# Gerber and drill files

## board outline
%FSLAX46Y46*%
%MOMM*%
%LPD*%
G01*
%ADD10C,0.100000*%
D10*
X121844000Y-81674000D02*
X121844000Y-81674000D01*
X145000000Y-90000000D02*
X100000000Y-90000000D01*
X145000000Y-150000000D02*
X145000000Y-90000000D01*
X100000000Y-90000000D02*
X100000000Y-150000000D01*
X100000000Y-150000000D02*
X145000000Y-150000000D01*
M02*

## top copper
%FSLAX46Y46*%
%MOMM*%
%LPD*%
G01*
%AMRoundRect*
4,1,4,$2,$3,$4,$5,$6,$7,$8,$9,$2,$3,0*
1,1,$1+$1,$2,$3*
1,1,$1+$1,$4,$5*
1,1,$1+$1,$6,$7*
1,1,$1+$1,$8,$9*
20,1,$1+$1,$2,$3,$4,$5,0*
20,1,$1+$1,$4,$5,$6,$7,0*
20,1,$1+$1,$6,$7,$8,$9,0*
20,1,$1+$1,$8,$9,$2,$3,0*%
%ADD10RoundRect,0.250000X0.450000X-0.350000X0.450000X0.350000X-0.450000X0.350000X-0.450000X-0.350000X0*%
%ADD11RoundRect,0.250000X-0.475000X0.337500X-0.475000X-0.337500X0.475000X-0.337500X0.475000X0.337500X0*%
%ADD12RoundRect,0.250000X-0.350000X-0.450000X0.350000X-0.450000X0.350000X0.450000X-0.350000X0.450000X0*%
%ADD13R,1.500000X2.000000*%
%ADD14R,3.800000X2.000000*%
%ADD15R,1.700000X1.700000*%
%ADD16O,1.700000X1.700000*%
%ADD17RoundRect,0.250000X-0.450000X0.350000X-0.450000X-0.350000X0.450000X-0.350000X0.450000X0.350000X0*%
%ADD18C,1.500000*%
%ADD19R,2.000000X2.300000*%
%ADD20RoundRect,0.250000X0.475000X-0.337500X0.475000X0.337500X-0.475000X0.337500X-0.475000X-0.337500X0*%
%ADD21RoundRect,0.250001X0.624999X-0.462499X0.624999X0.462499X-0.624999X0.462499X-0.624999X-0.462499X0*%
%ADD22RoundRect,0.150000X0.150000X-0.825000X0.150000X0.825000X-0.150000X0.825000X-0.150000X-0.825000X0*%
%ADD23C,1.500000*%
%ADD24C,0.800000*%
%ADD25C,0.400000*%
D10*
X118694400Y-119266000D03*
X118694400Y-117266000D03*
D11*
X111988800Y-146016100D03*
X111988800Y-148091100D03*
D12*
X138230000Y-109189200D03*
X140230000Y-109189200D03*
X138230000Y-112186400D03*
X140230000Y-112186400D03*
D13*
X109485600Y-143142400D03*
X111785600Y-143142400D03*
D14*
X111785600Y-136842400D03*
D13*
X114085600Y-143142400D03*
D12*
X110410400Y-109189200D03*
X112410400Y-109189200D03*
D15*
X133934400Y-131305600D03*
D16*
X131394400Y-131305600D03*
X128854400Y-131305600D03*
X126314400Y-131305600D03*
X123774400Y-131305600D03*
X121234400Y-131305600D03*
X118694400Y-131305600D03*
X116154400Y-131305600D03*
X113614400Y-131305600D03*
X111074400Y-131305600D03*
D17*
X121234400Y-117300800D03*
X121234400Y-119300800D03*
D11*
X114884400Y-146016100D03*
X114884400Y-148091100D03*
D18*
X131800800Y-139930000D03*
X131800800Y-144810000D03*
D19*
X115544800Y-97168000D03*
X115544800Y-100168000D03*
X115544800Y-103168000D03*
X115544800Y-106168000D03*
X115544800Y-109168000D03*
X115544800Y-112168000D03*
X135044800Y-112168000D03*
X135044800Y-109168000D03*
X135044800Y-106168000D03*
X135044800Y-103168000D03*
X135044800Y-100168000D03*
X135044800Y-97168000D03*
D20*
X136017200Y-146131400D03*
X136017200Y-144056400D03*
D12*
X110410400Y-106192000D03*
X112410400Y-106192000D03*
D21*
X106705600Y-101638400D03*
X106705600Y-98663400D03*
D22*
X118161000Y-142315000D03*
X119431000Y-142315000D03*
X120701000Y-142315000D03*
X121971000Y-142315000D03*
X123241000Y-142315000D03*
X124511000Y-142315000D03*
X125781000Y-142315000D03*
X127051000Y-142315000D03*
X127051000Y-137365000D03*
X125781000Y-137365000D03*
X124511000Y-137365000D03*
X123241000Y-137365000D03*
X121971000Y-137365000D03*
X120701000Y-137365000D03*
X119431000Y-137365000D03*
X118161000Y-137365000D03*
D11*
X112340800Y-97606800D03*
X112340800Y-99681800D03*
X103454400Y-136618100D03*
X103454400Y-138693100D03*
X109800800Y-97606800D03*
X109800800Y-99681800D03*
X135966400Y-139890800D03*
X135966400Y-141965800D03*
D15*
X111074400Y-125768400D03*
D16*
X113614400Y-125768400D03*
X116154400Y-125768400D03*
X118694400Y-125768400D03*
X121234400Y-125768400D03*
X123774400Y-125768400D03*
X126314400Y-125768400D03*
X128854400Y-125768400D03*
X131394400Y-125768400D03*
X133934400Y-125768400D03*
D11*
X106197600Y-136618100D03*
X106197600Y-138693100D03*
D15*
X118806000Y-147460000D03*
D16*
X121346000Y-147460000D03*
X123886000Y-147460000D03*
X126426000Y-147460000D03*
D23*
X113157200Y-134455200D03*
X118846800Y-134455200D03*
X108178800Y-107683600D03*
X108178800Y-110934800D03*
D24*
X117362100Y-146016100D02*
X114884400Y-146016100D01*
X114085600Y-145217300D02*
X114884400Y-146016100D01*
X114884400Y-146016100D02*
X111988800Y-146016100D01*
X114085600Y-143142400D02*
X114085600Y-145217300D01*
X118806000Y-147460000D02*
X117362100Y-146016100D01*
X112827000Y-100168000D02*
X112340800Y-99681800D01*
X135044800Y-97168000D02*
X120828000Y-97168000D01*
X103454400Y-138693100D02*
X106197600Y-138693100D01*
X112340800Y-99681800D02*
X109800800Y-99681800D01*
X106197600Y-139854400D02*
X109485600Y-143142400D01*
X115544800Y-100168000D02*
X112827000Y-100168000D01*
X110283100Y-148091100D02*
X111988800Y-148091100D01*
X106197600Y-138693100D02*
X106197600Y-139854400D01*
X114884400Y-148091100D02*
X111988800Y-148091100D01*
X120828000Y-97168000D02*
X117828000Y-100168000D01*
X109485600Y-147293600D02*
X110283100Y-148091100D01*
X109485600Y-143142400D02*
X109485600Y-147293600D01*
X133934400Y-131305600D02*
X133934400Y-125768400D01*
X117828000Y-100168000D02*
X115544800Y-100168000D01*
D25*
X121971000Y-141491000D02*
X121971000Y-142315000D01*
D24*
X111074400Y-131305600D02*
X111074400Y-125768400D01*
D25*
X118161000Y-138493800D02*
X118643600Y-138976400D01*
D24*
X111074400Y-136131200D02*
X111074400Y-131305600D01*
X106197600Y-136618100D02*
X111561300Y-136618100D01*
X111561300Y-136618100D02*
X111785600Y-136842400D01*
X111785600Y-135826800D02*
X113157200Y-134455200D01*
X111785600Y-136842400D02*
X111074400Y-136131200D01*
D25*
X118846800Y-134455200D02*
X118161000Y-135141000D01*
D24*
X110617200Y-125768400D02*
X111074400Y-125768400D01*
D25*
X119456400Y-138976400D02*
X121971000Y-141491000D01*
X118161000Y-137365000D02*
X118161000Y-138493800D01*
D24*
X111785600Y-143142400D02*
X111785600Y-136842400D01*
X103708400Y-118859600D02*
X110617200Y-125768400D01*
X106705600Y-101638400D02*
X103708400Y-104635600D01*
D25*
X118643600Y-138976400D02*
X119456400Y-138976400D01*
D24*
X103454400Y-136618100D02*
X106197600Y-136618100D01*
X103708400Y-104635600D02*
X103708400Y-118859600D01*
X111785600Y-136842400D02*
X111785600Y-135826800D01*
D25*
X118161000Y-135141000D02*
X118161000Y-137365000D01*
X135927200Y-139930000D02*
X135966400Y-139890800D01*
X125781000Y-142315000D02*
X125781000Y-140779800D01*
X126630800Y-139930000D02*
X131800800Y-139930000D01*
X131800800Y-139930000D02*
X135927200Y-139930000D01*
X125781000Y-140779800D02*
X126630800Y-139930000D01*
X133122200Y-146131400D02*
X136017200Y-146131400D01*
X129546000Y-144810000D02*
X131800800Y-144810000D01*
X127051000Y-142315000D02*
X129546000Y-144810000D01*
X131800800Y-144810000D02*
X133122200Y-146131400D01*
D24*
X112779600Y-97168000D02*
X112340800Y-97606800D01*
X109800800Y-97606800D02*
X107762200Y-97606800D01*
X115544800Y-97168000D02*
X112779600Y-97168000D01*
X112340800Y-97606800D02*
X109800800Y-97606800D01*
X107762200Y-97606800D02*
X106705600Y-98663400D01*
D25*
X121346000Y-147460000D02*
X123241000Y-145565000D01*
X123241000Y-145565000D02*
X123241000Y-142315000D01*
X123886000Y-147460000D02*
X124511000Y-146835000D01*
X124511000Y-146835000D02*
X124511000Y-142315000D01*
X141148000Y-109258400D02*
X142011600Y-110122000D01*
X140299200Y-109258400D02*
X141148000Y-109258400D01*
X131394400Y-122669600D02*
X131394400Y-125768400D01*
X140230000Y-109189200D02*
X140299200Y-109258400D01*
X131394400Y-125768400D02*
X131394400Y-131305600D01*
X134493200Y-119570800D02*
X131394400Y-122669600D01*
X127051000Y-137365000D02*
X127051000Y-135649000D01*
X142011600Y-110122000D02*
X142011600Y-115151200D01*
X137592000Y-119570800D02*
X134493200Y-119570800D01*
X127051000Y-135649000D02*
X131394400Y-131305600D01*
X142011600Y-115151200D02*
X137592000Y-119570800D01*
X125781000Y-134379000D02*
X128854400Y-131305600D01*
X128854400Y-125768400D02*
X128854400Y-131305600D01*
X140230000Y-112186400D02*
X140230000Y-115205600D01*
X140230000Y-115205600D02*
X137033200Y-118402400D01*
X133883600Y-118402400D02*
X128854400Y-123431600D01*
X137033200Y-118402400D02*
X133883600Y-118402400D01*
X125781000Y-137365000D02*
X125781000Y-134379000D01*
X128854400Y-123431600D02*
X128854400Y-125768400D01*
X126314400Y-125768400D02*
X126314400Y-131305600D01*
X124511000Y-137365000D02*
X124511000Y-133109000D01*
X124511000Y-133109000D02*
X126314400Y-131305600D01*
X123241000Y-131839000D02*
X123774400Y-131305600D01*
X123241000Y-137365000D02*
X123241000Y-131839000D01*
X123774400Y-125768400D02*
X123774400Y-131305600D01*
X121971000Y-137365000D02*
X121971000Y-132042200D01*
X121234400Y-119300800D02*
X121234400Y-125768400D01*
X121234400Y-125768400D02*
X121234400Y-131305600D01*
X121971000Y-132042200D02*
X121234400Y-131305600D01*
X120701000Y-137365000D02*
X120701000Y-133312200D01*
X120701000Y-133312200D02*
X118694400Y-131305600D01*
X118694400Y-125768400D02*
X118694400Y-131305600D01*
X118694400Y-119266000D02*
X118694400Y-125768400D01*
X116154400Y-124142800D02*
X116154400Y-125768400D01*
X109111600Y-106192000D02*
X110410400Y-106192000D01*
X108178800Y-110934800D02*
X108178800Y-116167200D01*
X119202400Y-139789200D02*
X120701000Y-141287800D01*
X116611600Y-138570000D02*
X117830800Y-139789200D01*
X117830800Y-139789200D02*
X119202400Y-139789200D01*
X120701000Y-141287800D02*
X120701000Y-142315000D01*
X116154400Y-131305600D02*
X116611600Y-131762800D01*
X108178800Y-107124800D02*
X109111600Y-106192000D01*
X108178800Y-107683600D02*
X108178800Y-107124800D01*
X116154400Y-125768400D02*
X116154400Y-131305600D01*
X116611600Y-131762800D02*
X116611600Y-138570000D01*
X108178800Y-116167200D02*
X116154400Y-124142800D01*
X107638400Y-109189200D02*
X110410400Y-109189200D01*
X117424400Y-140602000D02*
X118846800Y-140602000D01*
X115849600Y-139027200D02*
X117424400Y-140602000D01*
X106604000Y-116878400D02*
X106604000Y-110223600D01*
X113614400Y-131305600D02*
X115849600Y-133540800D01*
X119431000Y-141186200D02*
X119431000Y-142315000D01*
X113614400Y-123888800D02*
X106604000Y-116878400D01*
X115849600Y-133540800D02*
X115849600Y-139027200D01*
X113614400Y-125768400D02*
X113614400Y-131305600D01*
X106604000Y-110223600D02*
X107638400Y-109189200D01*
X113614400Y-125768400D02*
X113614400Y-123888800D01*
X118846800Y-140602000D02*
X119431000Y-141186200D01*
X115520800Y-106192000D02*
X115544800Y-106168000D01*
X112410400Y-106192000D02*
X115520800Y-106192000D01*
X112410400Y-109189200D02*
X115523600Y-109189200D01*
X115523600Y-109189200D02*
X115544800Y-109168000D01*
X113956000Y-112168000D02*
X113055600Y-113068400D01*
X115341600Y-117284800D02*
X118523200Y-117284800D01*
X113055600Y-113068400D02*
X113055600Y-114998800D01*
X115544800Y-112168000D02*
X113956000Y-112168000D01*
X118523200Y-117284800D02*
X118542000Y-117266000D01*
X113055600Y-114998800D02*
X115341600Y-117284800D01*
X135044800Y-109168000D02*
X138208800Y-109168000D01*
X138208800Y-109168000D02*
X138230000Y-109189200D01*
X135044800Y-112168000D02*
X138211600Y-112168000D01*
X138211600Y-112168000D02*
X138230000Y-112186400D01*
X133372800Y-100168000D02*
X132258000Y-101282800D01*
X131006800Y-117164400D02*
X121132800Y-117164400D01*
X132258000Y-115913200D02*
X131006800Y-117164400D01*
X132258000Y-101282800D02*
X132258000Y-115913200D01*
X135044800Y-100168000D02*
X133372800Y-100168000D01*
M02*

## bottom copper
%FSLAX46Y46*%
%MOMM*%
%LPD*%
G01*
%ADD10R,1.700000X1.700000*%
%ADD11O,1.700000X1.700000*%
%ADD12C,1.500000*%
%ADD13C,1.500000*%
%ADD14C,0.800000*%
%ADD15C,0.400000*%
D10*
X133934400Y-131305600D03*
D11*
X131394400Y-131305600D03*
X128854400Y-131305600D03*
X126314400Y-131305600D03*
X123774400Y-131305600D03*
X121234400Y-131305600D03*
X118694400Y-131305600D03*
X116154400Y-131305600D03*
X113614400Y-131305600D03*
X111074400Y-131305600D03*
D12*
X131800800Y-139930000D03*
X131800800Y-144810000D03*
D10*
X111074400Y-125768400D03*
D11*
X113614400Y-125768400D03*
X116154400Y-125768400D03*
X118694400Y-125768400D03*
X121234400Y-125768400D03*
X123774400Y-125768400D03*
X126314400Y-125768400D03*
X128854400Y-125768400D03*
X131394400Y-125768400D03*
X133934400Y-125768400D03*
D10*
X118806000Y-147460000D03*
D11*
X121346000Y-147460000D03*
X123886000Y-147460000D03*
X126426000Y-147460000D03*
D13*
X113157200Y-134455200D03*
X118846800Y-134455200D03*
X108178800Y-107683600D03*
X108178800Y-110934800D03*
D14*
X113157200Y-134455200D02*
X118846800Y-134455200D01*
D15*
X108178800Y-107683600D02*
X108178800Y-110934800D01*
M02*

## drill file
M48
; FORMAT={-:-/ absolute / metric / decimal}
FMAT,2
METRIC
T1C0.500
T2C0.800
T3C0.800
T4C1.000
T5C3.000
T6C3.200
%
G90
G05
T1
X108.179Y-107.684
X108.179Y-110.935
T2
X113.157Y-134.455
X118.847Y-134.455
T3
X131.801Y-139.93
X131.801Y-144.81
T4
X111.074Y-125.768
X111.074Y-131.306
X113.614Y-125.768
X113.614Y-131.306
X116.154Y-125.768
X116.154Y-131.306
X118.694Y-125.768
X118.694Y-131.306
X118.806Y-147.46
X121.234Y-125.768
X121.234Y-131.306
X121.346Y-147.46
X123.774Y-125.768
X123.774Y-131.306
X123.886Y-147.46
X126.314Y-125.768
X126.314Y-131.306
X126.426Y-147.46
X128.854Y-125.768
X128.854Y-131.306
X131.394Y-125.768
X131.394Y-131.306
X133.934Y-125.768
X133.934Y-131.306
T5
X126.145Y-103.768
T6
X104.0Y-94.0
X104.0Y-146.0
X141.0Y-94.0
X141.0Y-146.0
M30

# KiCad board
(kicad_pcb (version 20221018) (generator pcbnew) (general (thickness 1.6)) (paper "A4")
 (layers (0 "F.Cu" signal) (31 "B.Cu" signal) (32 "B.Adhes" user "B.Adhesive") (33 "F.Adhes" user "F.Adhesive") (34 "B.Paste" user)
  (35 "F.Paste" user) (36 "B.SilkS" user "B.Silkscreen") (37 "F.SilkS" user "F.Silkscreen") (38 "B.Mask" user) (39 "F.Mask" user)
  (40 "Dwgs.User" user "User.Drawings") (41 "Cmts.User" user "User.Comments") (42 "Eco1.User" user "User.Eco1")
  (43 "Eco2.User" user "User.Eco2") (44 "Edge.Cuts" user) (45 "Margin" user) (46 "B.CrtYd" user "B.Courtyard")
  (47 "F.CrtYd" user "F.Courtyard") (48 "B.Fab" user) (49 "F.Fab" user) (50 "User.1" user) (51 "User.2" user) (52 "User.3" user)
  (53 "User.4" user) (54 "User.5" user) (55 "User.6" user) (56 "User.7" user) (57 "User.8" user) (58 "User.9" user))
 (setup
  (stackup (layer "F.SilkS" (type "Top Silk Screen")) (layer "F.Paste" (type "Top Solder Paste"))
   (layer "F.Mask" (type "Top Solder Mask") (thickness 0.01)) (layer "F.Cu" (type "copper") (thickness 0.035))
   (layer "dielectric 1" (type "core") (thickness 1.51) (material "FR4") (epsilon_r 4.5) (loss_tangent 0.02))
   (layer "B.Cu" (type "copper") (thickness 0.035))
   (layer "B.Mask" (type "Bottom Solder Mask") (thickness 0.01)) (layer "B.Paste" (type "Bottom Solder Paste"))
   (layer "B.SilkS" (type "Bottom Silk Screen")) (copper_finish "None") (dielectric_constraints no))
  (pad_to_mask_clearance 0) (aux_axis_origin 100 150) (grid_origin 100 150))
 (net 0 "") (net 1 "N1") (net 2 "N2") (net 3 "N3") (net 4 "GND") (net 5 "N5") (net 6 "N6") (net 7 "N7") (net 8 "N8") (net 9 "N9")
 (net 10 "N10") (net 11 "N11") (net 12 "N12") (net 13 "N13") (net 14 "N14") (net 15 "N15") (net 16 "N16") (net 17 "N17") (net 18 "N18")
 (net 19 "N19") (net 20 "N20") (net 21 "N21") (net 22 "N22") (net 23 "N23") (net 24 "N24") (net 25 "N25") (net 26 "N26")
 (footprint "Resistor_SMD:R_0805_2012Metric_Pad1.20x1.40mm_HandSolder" (layer "F.Cu") (at 118.6944 118.266 90)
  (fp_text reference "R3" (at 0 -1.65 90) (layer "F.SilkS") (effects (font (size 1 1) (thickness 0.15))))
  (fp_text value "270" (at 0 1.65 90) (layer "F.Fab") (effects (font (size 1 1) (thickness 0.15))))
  (pad "1" smd roundrect (at -1 0 90) (size 1.2 1.4) (layers "F.Cu" "F.Paste" "F.Mask") (roundrect_rratio 0.208333) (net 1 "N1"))
  (pad "2" smd roundrect (at 1 0 90) (size 1.2 1.4) (layers "F.Cu" "F.Paste" "F.Mask") (roundrect_rratio 0.208333) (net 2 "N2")))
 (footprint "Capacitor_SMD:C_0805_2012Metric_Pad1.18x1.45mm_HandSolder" (layer "F.Cu") (at 111.9888 147.0536 -90)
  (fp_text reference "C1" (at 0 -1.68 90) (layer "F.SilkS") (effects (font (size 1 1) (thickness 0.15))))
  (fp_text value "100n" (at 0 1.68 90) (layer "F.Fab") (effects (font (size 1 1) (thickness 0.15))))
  (pad "1" smd roundrect (at -1.0375 0 270) (size 1.175 1.45) (layers "F.Cu" "F.Paste" "F.Mask") (roundrect_rratio 0.212766) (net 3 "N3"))
  (pad "2" smd roundrect (at 1.0375 0 270) (size 1.175 1.45) (layers "F.Cu" "F.Paste" "F.Mask") (roundrect_rratio 0.212766) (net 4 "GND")))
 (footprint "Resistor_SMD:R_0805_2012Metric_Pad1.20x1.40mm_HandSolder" (layer "F.Cu") (at 139.23 109.1892)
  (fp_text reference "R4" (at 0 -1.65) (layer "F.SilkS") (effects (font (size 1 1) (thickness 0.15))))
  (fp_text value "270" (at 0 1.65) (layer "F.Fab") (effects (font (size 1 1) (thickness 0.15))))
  (pad "1" smd roundrect (at -1 0) (size 1.2 1.4) (layers "F.Cu" "F.Paste" "F.Mask") (roundrect_rratio 0.208333) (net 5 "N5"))
  (pad "2" smd roundrect (at 1 0) (size 1.2 1.4) (layers "F.Cu" "F.Paste" "F.Mask") (roundrect_rratio 0.208333) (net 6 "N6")))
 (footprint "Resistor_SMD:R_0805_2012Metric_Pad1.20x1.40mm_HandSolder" (layer "F.Cu") (at 139.23 112.1864)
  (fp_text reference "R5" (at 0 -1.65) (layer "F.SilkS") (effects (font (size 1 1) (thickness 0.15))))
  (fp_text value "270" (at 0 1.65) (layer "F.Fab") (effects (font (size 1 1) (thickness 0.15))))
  (pad "1" smd roundrect (at -1 0) (size 1.2 1.4) (layers "F.Cu" "F.Paste" "F.Mask") (roundrect_rratio 0.208333) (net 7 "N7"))
  (pad "2" smd roundrect (at 1 0) (size 1.2 1.4) (layers "F.Cu" "F.Paste" "F.Mask") (roundrect_rratio 0.208333) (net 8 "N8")))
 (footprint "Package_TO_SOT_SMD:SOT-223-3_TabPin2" (layer "F.Cu") (at 111.7856 139.9924 90)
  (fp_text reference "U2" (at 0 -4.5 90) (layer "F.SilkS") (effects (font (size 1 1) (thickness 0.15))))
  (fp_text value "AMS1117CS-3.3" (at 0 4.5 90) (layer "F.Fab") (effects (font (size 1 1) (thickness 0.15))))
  (pad "1" smd rect (at -3.15 -2.3 90) (size 2 1.5) (layers "F.Cu" "F.Paste" "F.Mask") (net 4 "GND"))
  (pad "2" smd rect (at -3.15 0 90) (size 2 1.5) (layers "F.Cu" "F.Paste" "F.Mask") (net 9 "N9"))
  (pad "2" smd rect (at 3.15 0 90) (size 2 3.8) (layers "F.Cu" "F.Paste" "F.Mask") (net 9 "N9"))
  (pad "3" smd rect (at -3.15 2.3 90) (size 2 1.5) (layers "F.Cu" "F.Paste" "F.Mask") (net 3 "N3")))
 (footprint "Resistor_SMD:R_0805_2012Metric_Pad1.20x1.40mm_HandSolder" (layer "F.Cu") (at 111.4104 109.1892)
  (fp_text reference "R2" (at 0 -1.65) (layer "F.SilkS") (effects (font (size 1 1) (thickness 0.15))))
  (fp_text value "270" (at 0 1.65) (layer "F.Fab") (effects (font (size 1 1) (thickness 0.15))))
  (pad "1" smd roundrect (at -1 0) (size 1.2 1.4) (layers "F.Cu" "F.Paste" "F.Mask") (roundrect_rratio 0.208333) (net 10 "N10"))
  (pad "2" smd roundrect (at 1 0) (size 1.2 1.4) (layers "F.Cu" "F.Paste" "F.Mask") (roundrect_rratio 0.208333) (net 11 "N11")))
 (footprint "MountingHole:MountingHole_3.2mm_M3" (layer "F.Cu") (at 141 146)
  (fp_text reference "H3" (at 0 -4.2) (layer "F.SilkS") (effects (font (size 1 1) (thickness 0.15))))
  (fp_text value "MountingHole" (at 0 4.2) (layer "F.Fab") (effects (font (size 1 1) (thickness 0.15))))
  (pad "" np_thru_hole circle (at 0 0) (size 3.2 3.2) (drill 3.2) (layers "*.Cu" "*.Mask")))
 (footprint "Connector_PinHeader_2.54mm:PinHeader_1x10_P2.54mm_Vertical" (layer "F.Cu") (at 133.9344 131.3056 -90)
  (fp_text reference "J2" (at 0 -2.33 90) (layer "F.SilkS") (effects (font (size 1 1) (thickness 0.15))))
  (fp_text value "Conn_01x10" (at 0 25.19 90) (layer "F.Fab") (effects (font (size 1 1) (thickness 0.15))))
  (pad "1" thru_hole rect (at 0 0 270) (size 1.7 1.7) (drill 1) (layers "*.Cu" "*.Mask") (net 4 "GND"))
  (pad "2" thru_hole oval (at 0 2.54 270) (size 1.7 1.7) (drill 1) (layers "*.Cu" "*.Mask") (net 6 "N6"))
  (pad "3" thru_hole oval (at 0 5.08 270) (size 1.7 1.7) (drill 1) (layers "*.Cu" "*.Mask") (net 8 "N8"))
  (pad "4" thru_hole oval (at 0 7.62 270) (size 1.7 1.7) (drill 1) (layers "*.Cu" "*.Mask") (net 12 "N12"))
  (pad "5" thru_hole oval (at 0 10.16 270) (size 1.7 1.7) (drill 1) (layers "*.Cu" "*.Mask") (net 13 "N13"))
  (pad "6" thru_hole oval (at 0 12.7 270) (size 1.7 1.7) (drill 1) (layers "*.Cu" "*.Mask") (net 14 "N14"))
  (pad "7" thru_hole oval (at 0 15.24 270) (size 1.7 1.7) (drill 1) (layers "*.Cu" "*.Mask") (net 1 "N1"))
  (pad "8" thru_hole oval (at 0 17.78 270) (size 1.7 1.7) (drill 1) (layers "*.Cu" "*.Mask") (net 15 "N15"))
  (pad "9" thru_hole oval (at 0 20.32 270) (size 1.7 1.7) (drill 1) (layers "*.Cu" "*.Mask") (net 10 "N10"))
  (pad "10" thru_hole oval (at 0 22.86 270) (size 1.7 1.7) (drill 1) (layers "*.Cu" "*.Mask") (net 9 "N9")))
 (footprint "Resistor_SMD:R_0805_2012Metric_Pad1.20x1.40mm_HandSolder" (layer "F.Cu") (at 121.2344 118.3008 -90)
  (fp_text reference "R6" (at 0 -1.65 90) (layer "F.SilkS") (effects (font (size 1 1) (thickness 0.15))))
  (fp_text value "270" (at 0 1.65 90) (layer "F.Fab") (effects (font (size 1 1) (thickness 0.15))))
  (pad "1" smd roundrect (at -1 0 270) (size 1.2 1.4) (layers "F.Cu" "F.Paste" "F.Mask") (roundrect_rratio 0.208333) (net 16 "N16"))
  (pad "2" smd roundrect (at 1 0 270) (size 1.2 1.4) (layers "F.Cu" "F.Paste" "F.Mask") (roundrect_rratio 0.208333) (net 14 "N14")))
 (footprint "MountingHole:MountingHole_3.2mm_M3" (layer "F.Cu") (at 104 94)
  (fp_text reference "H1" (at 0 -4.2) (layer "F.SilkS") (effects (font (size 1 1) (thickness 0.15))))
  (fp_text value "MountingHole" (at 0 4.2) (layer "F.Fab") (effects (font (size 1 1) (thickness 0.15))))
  (pad "" np_thru_hole circle (at 0 0) (size 3.2 3.2) (drill 3.2) (layers "*.Cu" "*.Mask")))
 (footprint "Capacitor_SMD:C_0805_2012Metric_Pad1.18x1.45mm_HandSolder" (layer "F.Cu") (at 114.8844 147.0536 -90)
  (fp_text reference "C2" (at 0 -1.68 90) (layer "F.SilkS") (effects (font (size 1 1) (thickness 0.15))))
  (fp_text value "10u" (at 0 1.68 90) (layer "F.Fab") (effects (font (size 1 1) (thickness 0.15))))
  (pad "1" smd roundrect (at -1.0375 0 270) (size 1.175 1.45) (layers "F.Cu" "F.Paste" "F.Mask") (roundrect_rratio 0.212766) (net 3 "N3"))
  (pad "2" smd roundrect (at 1.0375 0 270) (size 1.175 1.45) (layers "F.Cu" "F.Paste" "F.Mask") (roundrect_rratio 0.212766) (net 4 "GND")))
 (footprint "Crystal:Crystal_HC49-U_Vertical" (layer "F.Cu") (at 131.8008 139.93 -90)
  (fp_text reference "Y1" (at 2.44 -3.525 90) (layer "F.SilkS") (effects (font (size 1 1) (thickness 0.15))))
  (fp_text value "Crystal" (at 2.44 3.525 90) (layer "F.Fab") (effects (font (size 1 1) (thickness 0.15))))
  (pad "1" thru_hole circle (at 0 0 270) (size 1.5 1.5) (drill 0.8) (layers "*.Cu" "*.Mask") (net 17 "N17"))
  (pad "2" thru_hole circle (at 4.88 0 270) (size 1.5 1.5) (drill 0.8) (layers "*.Cu" "*.Mask") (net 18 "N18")))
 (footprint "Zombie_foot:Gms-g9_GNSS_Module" (layer "F.Cu") (at 125.2948 104.668)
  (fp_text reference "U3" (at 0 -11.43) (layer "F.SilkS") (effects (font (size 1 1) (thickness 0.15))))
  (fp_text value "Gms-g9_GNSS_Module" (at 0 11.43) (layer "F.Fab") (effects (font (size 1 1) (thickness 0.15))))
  (pad "" np_thru_hole circle (at 0.85 -0.9) (size 3 3) (drill 3) (layers "*.Cu" "*.Mask"))
  (pad "1" smd rect (at -9.75 -7.5) (size 2 2.3) (layers "F.Cu" "F.Paste" "F.Mask") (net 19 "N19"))
  (pad "2" smd rect (at -9.75 -4.5) (size 2 2.3) (layers "F.Cu" "F.Paste" "F.Mask") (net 4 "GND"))
  (pad "3" smd rect (at -9.75 -1.5) (size 2 2.3) (layers "F.Cu" "F.Paste" "F.Mask") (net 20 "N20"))
  (pad "4" smd rect (at -9.75 1.5) (size 2 2.3) (layers "F.Cu" "F.Paste" "F.Mask") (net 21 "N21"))
  (pad "5" smd rect (at -9.75 4.5) (size 2 2.3) (layers "F.Cu" "F.Paste" "F.Mask") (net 11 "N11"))
  (pad "6" smd rect (at -9.75 7.5) (size 2 2.3) (layers "F.Cu" "F.Paste" "F.Mask") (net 2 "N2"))
  (pad "7" smd rect (at 9.75 7.5) (size 2 2.3) (layers "F.Cu" "F.Paste" "F.Mask") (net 7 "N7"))
  (pad "8" smd rect (at 9.75 4.5) (size 2 2.3) (layers "F.Cu" "F.Paste" "F.Mask") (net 5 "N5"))
  (pad "9" smd rect (at 9.75 1.5) (size 2 2.3) (layers "F.Cu" "F.Paste" "F.Mask") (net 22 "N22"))
  (pad "10" smd rect (at 9.75 -1.5) (size 2 2.3) (layers "F.Cu" "F.Paste" "F.Mask") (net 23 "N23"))
  (pad "11" smd rect (at 9.75 -4.5) (size 2 2.3) (layers "F.Cu" "F.Paste" "F.Mask") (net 16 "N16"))
  (pad "12" smd rect (at 9.75 -7.5) (size 2 2.3) (layers "F.Cu" "F.Paste" "F.Mask") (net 4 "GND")))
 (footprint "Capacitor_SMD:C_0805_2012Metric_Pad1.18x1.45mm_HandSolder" (layer "F.Cu") (at 136.0172 145.0939 90)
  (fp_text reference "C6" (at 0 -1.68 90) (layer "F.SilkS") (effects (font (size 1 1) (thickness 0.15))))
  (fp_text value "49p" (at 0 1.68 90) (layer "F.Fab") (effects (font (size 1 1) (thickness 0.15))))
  (pad "1" smd roundrect (at -1.0375 0 90) (size 1.175 1.45) (layers "F.Cu" "F.Paste" "F.Mask") (roundrect_rratio 0.212766) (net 18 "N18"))
  (pad "2" smd roundrect (at 1.0375 0 90) (size 1.175 1.45) (layers "F.Cu" "F.Paste" "F.Mask") (roundrect_rratio 0.212766) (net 4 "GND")))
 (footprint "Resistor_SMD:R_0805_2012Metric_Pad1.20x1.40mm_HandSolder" (layer "F.Cu") (at 111.4104 106.192)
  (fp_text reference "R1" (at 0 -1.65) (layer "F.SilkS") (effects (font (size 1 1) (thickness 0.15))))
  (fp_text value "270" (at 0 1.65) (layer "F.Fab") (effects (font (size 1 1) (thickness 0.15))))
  (pad "1" smd roundrect (at -1 0) (size 1.2 1.4) (layers "F.Cu" "F.Paste" "F.Mask") (roundrect_rratio 0.208333) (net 15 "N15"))
  (pad "2" smd roundrect (at 1 0) (size 1.2 1.4) (layers "F.Cu" "F.Paste" "F.Mask") (roundrect_rratio 0.208333) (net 21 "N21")))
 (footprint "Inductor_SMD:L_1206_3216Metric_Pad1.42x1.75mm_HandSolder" (layer "F.Cu") (at 106.7056 100.1509 90)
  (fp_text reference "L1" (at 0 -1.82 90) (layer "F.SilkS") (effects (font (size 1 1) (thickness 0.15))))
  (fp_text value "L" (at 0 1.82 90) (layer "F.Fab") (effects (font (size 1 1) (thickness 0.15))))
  (pad "1" smd roundrect (at -1.4875 0 90) (size 1.425 1.75) (layers "F.Cu" "F.Paste" "F.Mask") (roundrect_rratio 0.175439) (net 9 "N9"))
  (pad "2" smd roundrect (at 1.4875 0 90) (size 1.425 1.75) (layers "F.Cu" "F.Paste" "F.Mask") (roundrect_rratio 0.175439) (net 19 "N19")))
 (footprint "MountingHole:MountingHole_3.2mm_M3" (layer "F.Cu") (at 141 94)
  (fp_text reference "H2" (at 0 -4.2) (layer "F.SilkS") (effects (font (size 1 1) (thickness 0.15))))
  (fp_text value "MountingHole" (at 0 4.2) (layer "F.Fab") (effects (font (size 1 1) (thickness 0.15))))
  (pad "" np_thru_hole circle (at 0 0) (size 3.2 3.2) (drill 3.2) (layers "*.Cu" "*.Mask")))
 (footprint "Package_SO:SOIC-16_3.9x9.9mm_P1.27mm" (layer "F.Cu") (at 122.606 139.84 90)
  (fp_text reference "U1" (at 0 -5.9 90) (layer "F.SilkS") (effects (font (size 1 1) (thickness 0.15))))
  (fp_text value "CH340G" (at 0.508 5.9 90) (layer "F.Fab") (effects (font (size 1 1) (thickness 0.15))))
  (pad "1" smd roundrect (at -2.475 -4.445 90) (size 1.95 0.6) (layers "F.Cu" "F.Paste" "F.Mask") (roundrect_rratio 0.25) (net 4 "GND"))
  (pad "2" smd roundrect (at -2.475 -3.175 90) (size 1.95 0.6) (layers "F.Cu" "F.Paste" "F.Mask") (roundrect_rratio 0.25) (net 10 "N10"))
  (pad "3" smd roundrect (at -2.475 -1.905 90) (size 1.95 0.6) (layers "F.Cu" "F.Paste" "F.Mask") (roundrect_rratio 0.25) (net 15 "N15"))
  (pad "4" smd roundrect (at -2.475 -0.635 90) (size 1.95 0.6) (layers "F.Cu" "F.Paste" "F.Mask") (roundrect_rratio 0.25) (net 9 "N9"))
  (pad "5" smd roundrect (at -2.475 0.635 90) (size 1.95 0.6) (layers "F.Cu" "F.Paste" "F.Mask") (roundrect_rratio 0.25) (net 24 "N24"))
  (pad "6" smd roundrect (at -2.475 1.905 90) (size 1.95 0.6) (layers "F.Cu" "F.Paste" "F.Mask") (roundrect_rratio 0.25) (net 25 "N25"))
  (pad "7" smd roundrect (at -2.475 3.175 90) (size 1.95 0.6) (layers "F.Cu" "F.Paste" "F.Mask") (roundrect_rratio 0.25) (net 17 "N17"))
  (pad "8" smd roundrect (at -2.475 4.445 90) (size 1.95 0.6) (layers "F.Cu" "F.Paste" "F.Mask") (roundrect_rratio 0.25) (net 18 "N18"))
  (pad "9" smd roundrect (at 2.475 4.445 90) (size 1.95 0.6) (layers "F.Cu" "F.Paste" "F.Mask") (roundrect_rratio 0.25) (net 6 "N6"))
  (pad "10" smd roundrect (at 2.475 3.175 90) (size 1.95 0.6) (layers "F.Cu" "F.Paste" "F.Mask") (roundrect_rratio 0.25) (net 8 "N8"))
  (pad "11" smd roundrect (at 2.475 1.905 90) (size 1.95 0.6) (layers "F.Cu" "F.Paste" "F.Mask") (roundrect_rratio 0.25) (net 12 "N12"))
  (pad "12" smd roundrect (at 2.475 0.635 90) (size 1.95 0.6) (layers "F.Cu" "F.Paste" "F.Mask") (roundrect_rratio 0.25) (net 13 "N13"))
  (pad "13" smd roundrect (at 2.475 -0.635 90) (size 1.95 0.6) (layers "F.Cu" "F.Paste" "F.Mask") (roundrect_rratio 0.25) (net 14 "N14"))
  (pad "14" smd roundrect (at 2.475 -1.905 90) (size 1.95 0.6) (layers "F.Cu" "F.Paste" "F.Mask") (roundrect_rratio 0.25) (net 1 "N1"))
  (pad "15" smd roundrect (at 2.475 -3.175 90) (size 1.95 0.6) (layers "F.Cu" "F.Paste" "F.Mask") (roundrect_rratio 0.25) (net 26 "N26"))
  (pad "16" smd roundrect (at 2.475 -4.445 90) (size 1.95 0.6) (layers "F.Cu" "F.Paste" "F.Mask") (roundrect_rratio 0.25) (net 9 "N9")))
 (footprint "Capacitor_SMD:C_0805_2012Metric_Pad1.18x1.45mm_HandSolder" (layer "F.Cu") (at 112.3408 98.6443 -90)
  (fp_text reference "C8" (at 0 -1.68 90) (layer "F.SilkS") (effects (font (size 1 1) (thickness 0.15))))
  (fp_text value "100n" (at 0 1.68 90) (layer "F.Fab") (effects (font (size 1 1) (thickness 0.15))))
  (pad "1" smd roundrect (at -1.0375 0 270) (size 1.175 1.45) (layers "F.Cu" "F.Paste" "F.Mask") (roundrect_rratio 0.212766) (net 19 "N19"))
  (pad "2" smd roundrect (at 1.0375 0 270) (size 1.175 1.45) (layers "F.Cu" "F.Paste" "F.Mask") (roundrect_rratio 0.212766) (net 4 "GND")))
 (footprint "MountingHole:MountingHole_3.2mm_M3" (layer "F.Cu") (at 104 146)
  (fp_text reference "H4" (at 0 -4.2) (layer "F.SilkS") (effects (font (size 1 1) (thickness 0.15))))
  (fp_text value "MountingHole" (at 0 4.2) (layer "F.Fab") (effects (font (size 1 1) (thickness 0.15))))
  (pad "" np_thru_hole circle (at 0 0) (size 3.2 3.2) (drill 3.2) (layers "*.Cu" "*.Mask")))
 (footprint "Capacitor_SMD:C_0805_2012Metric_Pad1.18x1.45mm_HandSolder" (layer "F.Cu") (at 103.4544 137.6556 -90)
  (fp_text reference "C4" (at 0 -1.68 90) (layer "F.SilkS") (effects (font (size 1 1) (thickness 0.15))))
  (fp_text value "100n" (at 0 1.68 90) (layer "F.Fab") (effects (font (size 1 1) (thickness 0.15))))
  (pad "1" smd roundrect (at -1.0375 0 270) (size 1.175 1.45) (layers "F.Cu" "F.Paste" "F.Mask") (roundrect_rratio 0.212766) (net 9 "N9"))
  (pad "2" smd roundrect (at 1.0375 0 270) (size 1.175 1.45) (layers "F.Cu" "F.Paste" "F.Mask") (roundrect_rratio 0.212766) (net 4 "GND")))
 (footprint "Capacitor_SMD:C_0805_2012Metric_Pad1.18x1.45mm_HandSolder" (layer "F.Cu") (at 109.8008 98.6443 -90)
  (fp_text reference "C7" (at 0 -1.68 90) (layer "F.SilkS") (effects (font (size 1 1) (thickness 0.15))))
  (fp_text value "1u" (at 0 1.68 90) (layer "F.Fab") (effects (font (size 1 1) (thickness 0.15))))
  (pad "1" smd roundrect (at -1.0375 0 270) (size 1.175 1.45) (layers "F.Cu" "F.Paste" "F.Mask") (roundrect_rratio 0.212766) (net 19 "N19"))
  (pad "2" smd roundrect (at 1.0375 0 270) (size 1.175 1.45) (layers "F.Cu" "F.Paste" "F.Mask") (roundrect_rratio 0.212766) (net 4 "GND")))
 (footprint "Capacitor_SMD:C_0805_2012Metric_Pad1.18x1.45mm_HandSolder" (layer "F.Cu") (at 135.9664 140.9283 -90)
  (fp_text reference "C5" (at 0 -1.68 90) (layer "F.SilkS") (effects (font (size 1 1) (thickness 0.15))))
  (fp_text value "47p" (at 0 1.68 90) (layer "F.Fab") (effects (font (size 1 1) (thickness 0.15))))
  (pad "1" smd roundrect (at -1.0375 0 270) (size 1.175 1.45) (layers "F.Cu" "F.Paste" "F.Mask") (roundrect_rratio 0.212766) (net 17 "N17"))
  (pad "2" smd roundrect (at 1.0375 0 270) (size 1.175 1.45) (layers "F.Cu" "F.Paste" "F.Mask") (roundrect_rratio 0.212766) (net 4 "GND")))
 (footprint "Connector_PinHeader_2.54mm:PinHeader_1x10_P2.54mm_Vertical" (layer "F.Cu") (at 111.0744 125.7684 90)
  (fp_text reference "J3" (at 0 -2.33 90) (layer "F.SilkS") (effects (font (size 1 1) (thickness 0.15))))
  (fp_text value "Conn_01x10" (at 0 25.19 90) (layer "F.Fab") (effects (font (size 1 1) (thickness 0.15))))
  (pad "1" thru_hole rect (at 0 0 90) (size 1.7 1.7) (drill 1) (layers "*.Cu" "*.Mask") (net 9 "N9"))
  (pad "2" thru_hole oval (at 0 2.54 90) (size 1.7 1.7) (drill 1) (layers "*.Cu" "*.Mask") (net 10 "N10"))
  (pad "3" thru_hole oval (at 0 5.08 90) (size 1.7 1.7) (drill 1) (layers "*.Cu" "*.Mask") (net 15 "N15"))
  (pad "4" thru_hole oval (at 0 7.62 90) (size 1.7 1.7) (drill 1) (layers "*.Cu" "*.Mask") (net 1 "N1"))
  (pad "5" thru_hole oval (at 0 10.16 90) (size 1.7 1.7) (drill 1) (layers "*.Cu" "*.Mask") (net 14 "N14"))
  (pad "6" thru_hole oval (at 0 12.7 90) (size 1.7 1.7) (drill 1) (layers "*.Cu" "*.Mask") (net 13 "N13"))
  (pad "7" thru_hole oval (at 0 15.24 90) (size 1.7 1.7) (drill 1) (layers "*.Cu" "*.Mask") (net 12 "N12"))
  (pad "8" thru_hole oval (at 0 17.78 90) (size 1.7 1.7) (drill 1) (layers "*.Cu" "*.Mask") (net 8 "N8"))
  (pad "9" thru_hole oval (at 0 20.32 90) (size 1.7 1.7) (drill 1) (layers "*.Cu" "*.Mask") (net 6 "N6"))
  (pad "10" thru_hole oval (at 0 22.86 90) (size 1.7 1.7) (drill 1) (layers "*.Cu" "*.Mask") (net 4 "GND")))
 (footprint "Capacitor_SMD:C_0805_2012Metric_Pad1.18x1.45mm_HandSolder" (layer "F.Cu") (at 106.1976 137.6556 -90)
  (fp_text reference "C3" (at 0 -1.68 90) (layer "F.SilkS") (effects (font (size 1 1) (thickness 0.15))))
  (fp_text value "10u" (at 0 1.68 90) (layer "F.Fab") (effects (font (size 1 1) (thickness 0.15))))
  (pad "1" smd roundrect (at -1.0375 0 270) (size 1.175 1.45) (layers "F.Cu" "F.Paste" "F.Mask") (roundrect_rratio 0.212766) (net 9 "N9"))
  (pad "2" smd roundrect (at 1.0375 0 270) (size 1.175 1.45) (layers "F.Cu" "F.Paste" "F.Mask") (roundrect_rratio 0.212766) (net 4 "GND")))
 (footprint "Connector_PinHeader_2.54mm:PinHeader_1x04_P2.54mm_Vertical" (layer "F.Cu") (at 118.806 147.46 90)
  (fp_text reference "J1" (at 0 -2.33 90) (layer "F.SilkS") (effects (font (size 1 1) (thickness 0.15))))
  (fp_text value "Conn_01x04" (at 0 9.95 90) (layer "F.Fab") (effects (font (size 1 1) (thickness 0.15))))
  (pad "1" thru_hole rect (at 0 0 90) (size 1.7 1.7) (drill 1) (layers "*.Cu" "*.Mask") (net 3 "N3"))
  (pad "2" thru_hole oval (at 0 2.54 90) (size 1.7 1.7) (drill 1) (layers "*.Cu" "*.Mask") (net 24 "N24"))
  (pad "3" thru_hole oval (at 0 5.08 90) (size 1.7 1.7) (drill 1) (layers "*.Cu" "*.Mask") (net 25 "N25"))
  (pad "4" thru_hole oval (at 0 7.62 90) (size 1.7 1.7) (drill 1) (layers "*.Cu" "*.Mask") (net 4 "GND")))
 (gr_line (start 121.844 81.674) (end 121.844 81.674) (stroke (width 0.1) (type default)) (layer "Edge.Cuts"))
 (gr_line (start 145 90) (end 100 90) (stroke (width 0.1) (type default)) (layer "Edge.Cuts"))
 (gr_line (start 145 150) (end 145 90) (stroke (width 0.1) (type default)) (layer "Edge.Cuts"))
 (gr_line (start 100 90) (end 100 150) (stroke (width 0.1) (type default)) (layer "Edge.Cuts"))
 (gr_line (start 100 150) (end 145 150) (stroke (width 0.1) (type default)) (layer "Edge.Cuts"))
 (segment (start 117.3621 146.0161) (end 114.8844 146.0161) (width 0.8) (layer "F.Cu") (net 3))
 (segment (start 114.0856 145.2173) (end 114.8844 146.0161) (width 0.8) (layer "F.Cu") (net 3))
 (segment (start 114.8844 146.0161) (end 111.9888 146.0161) (width 0.8) (layer "F.Cu") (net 3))
 (segment (start 114.0856 143.1424) (end 114.0856 145.2173) (width 0.8) (layer "F.Cu") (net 3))
 (segment (start 118.806 147.46) (end 117.3621 146.0161) (width 0.8) (layer "F.Cu") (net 3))
 (segment (start 112.827 100.168) (end 112.3408 99.6818) (width 0.8) (layer "F.Cu") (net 4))
 (segment (start 135.0448 97.168) (end 120.828 97.168) (width 0.8) (layer "F.Cu") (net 4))
 (segment (start 103.4544 138.6931) (end 106.1976 138.6931) (width 0.8) (layer "F.Cu") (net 4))
 (segment (start 112.3408 99.6818) (end 109.8008 99.6818) (width 0.8) (layer "F.Cu") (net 4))
 (segment (start 106.1976 139.8544) (end 109.4856 143.1424) (width 0.8) (layer "F.Cu") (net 4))
 (segment (start 115.5448 100.168) (end 112.827 100.168) (width 0.8) (layer "F.Cu") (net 4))
 (segment (start 110.2831 148.0911) (end 111.9888 148.0911) (width 0.8) (layer "F.Cu") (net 4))
 (segment (start 106.1976 138.6931) (end 106.1976 139.8544) (width 0.8) (layer "F.Cu") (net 4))
 (segment (start 114.8844 148.0911) (end 111.9888 148.0911) (width 0.8) (layer "F.Cu") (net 4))
 (segment (start 120.828 97.168) (end 117.828 100.168) (width 0.8) (layer "F.Cu") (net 4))
 (segment (start 109.4856 147.2936) (end 110.2831 148.0911) (width 0.8) (layer "F.Cu") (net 4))
 (segment (start 109.4856 143.1424) (end 109.4856 147.2936) (width 0.8) (layer "F.Cu") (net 4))
 (segment (start 133.9344 131.3056) (end 133.9344 125.7684) (width 0.8) (layer "F.Cu") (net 4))
 (segment (start 117.828 100.168) (end 115.5448 100.168) (width 0.8) (layer "F.Cu") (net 4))
 (segment (start 121.971 141.491) (end 121.971 142.315) (width 0.4) (layer "F.Cu") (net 9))
 (segment (start 111.0744 131.3056) (end 111.0744 125.7684) (width 0.8) (layer "F.Cu") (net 9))
 (segment (start 118.161 138.4938) (end 118.6436 138.9764) (width 0.4) (layer "F.Cu") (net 9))
 (segment (start 111.0744 136.1312) (end 111.0744 131.3056) (width 0.8) (layer "F.Cu") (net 9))
 (segment (start 106.1976 136.6181) (end 111.5613 136.6181) (width 0.8) (layer "F.Cu") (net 9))
 (segment (start 111.5613 136.6181) (end 111.7856 136.8424) (width 0.8) (layer "F.Cu") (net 9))
 (segment (start 111.7856 135.8268) (end 113.1572 134.4552) (width 0.8) (layer "F.Cu") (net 9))
 (segment (start 111.7856 136.8424) (end 111.0744 136.1312) (width 0.8) (layer "F.Cu") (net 9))
 (segment (start 118.8468 134.4552) (end 118.161 135.141) (width 0.4) (layer "F.Cu") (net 9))
 (segment (start 110.6172 125.7684) (end 111.0744 125.7684) (width 0.8) (layer "F.Cu") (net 9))
 (segment (start 119.4564 138.9764) (end 121.971 141.491) (width 0.4) (layer "F.Cu") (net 9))
 (segment (start 118.161 137.365) (end 118.161 138.4938) (width 0.4) (layer "F.Cu") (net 9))
 (segment (start 111.7856 143.1424) (end 111.7856 136.8424) (width 0.8) (layer "F.Cu") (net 9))
 (segment (start 103.7084 118.8596) (end 110.6172 125.7684) (width 0.8) (layer "F.Cu") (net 9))
 (segment (start 106.7056 101.6384) (end 103.7084 104.6356) (width 0.8) (layer "F.Cu") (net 9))
 (segment (start 118.6436 138.9764) (end 119.4564 138.9764) (width 0.4) (layer "F.Cu") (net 9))
 (segment (start 103.4544 136.6181) (end 106.1976 136.6181) (width 0.8) (layer "F.Cu") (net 9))
 (segment (start 103.7084 104.6356) (end 103.7084 118.8596) (width 0.8) (layer "F.Cu") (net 9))
 (segment (start 111.7856 136.8424) (end 111.7856 135.8268) (width 0.8) (layer "F.Cu") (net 9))
 (segment (start 118.161 135.141) (end 118.161 137.365) (width 0.4) (layer "F.Cu") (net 9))
 (via (at 113.1572 134.4552) (size 1.5) (drill 0.8) (layers "F.Cu" "B.Cu") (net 9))
 (via (at 118.8468 134.4552) (size 1.5) (drill 0.8) (layers "F.Cu" "B.Cu") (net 9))
 (segment (start 113.1572 134.4552) (end 118.8468 134.4552) (width 0.8) (layer "B.Cu") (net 9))
 (segment (start 135.9272 139.93) (end 135.9664 139.8908) (width 0.4) (layer "F.Cu") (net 17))
 (segment (start 125.781 142.315) (end 125.781 140.7798) (width 0.4) (layer "F.Cu") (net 17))
 (segment (start 126.6308 139.93) (end 131.8008 139.93) (width 0.4) (layer "F.Cu") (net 17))
 (segment (start 131.8008 139.93) (end 135.9272 139.93) (width 0.4) (layer "F.Cu") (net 17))
 (segment (start 125.781 140.7798) (end 126.6308 139.93) (width 0.4) (layer "F.Cu") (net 17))
 (segment (start 133.1222 146.1314) (end 136.0172 146.1314) (width 0.4) (layer "F.Cu") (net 18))
 (segment (start 129.546 144.81) (end 131.8008 144.81) (width 0.4) (layer "F.Cu") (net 18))
 (segment (start 127.051 142.315) (end 129.546 144.81) (width 0.4) (layer "F.Cu") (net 18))
 (segment (start 131.8008 144.81) (end 133.1222 146.1314) (width 0.4) (layer "F.Cu") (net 18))
 (segment (start 112.7796 97.168) (end 112.3408 97.6068) (width 0.8) (layer "F.Cu") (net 19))
 (segment (start 109.8008 97.6068) (end 107.7622 97.6068) (width 0.8) (layer "F.Cu") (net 19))
 (segment (start 115.5448 97.168) (end 112.7796 97.168) (width 0.8) (layer "F.Cu") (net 19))
 (segment (start 112.3408 97.6068) (end 109.8008 97.6068) (width 0.8) (layer "F.Cu") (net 19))
 (segment (start 107.7622 97.6068) (end 106.7056 98.6634) (width 0.8) (layer "F.Cu") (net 19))
 (segment (start 121.346 147.46) (end 123.241 145.565) (width 0.4) (layer "F.Cu") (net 24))
 (segment (start 123.241 145.565) (end 123.241 142.315) (width 0.4) (layer "F.Cu") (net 24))
 (segment (start 123.886 147.46) (end 124.511 146.835) (width 0.4) (layer "F.Cu") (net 25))
 (segment (start 124.511 146.835) (end 124.511 142.315) (width 0.4) (layer "F.Cu") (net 25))
 (segment (start 141.148 109.2584) (end 142.0116 110.122) (width 0.4) (layer "F.Cu") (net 6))
 (segment (start 140.2992 109.2584) (end 141.148 109.2584) (width 0.4) (layer "F.Cu") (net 6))
 (segment (start 131.3944 122.6696) (end 131.3944 125.7684) (width 0.4) (layer "F.Cu") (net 6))
 (segment (start 140.23 109.1892) (end 140.2992 109.2584) (width 0.4) (layer "F.Cu") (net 6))
 (segment (start 131.3944 125.7684) (end 131.3944 131.3056) (width 0.4) (layer "F.Cu") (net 6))
 (segment (start 134.4932 119.5708) (end 131.3944 122.6696) (width 0.4) (layer "F.Cu") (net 6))
 (segment (start 127.051 137.365) (end 127.051 135.649) (width 0.4) (layer "F.Cu") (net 6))
 (segment (start 142.0116 110.122) (end 142.0116 115.1512) (width 0.4) (layer "F.Cu") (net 6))
 (segment (start 137.592 119.5708) (end 134.4932 119.5708) (width 0.4) (layer "F.Cu") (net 6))
 (segment (start 127.051 135.649) (end 131.3944 131.3056) (width 0.4) (layer "F.Cu") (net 6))
 (segment (start 142.0116 115.1512) (end 137.592 119.5708) (width 0.4) (layer "F.Cu") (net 6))
 (segment (start 125.781 134.379) (end 128.8544 131.3056) (width 0.4) (layer "F.Cu") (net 8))
 (segment (start 128.8544 125.7684) (end 128.8544 131.3056) (width 0.4) (layer "F.Cu") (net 8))
 (segment (start 140.23 112.1864) (end 140.23 115.2056) (width 0.4) (layer "F.Cu") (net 8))
 (segment (start 140.23 115.2056) (end 137.0332 118.4024) (width 0.4) (layer "F.Cu") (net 8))
 (segment (start 133.8836 118.4024) (end 128.8544 123.4316) (width 0.4) (layer "F.Cu") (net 8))
 (segment (start 137.0332 118.4024) (end 133.8836 118.4024) (width 0.4) (layer "F.Cu") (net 8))
 (segment (start 125.781 137.365) (end 125.781 134.379) (width 0.4) (layer "F.Cu") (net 8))
 (segment (start 128.8544 123.4316) (end 128.8544 125.7684) (width 0.4) (layer "F.Cu") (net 8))
 (segment (start 126.3144 125.7684) (end 126.3144 131.3056) (width 0.4) (layer "F.Cu") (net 12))
 (segment (start 124.511 137.365) (end 124.511 133.109) (width 0.4) (layer "F.Cu") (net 12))
 (segment (start 124.511 133.109) (end 126.3144 131.3056) (width 0.4) (layer "F.Cu") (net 12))
 (segment (start 123.241 131.839) (end 123.7744 131.3056) (width 0.4) (layer "F.Cu") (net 13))
 (segment (start 123.241 137.365) (end 123.241 131.839) (width 0.4) (layer "F.Cu") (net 13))
 (segment (start 123.7744 125.7684) (end 123.7744 131.3056) (width 0.4) (layer "F.Cu") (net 13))
 (segment (start 121.971 137.365) (end 121.971 132.0422) (width 0.4) (layer "F.Cu") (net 14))
 (segment (start 121.2344 119.3008) (end 121.2344 125.7684) (width 0.4) (layer "F.Cu") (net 14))
 (segment (start 121.2344 125.7684) (end 121.2344 131.3056) (width 0.4) (layer "F.Cu") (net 14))
 (segment (start 121.971 132.0422) (end 121.2344 131.3056) (width 0.4) (layer "F.Cu") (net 14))
 (segment (start 120.701 137.365) (end 120.701 133.3122) (width 0.4) (layer "F.Cu") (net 1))
 (segment (start 120.701 133.3122) (end 118.6944 131.3056) (width 0.4) (layer "F.Cu") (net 1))
 (segment (start 118.6944 125.7684) (end 118.6944 131.3056) (width 0.4) (layer "F.Cu") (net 1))
 (segment (start 118.6944 119.266) (end 118.6944 125.7684) (width 0.4) (layer "F.Cu") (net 1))
 (segment (start 116.1544 124.1428) (end 116.1544 125.7684) (width 0.4) (layer "F.Cu") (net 15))
 (segment (start 109.1116 106.192) (end 110.4104 106.192) (width 0.4) (layer "F.Cu") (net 15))
 (segment (start 108.1788 110.9348) (end 108.1788 116.1672) (width 0.4) (layer "F.Cu") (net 15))
 (segment (start 119.2024 139.7892) (end 120.701 141.2878) (width 0.4) (layer "F.Cu") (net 15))
 (segment (start 116.6116 138.57) (end 117.8308 139.7892) (width 0.4) (layer "F.Cu") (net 15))
 (segment (start 117.8308 139.7892) (end 119.2024 139.7892) (width 0.4) (layer "F.Cu") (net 15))
 (segment (start 120.701 141.2878) (end 120.701 142.315) (width 0.4) (layer "F.Cu") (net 15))
 (segment (start 116.1544 131.3056) (end 116.6116 131.7628) (width 0.4) (layer "F.Cu") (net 15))
 (segment (start 108.1788 107.1248) (end 109.1116 106.192) (width 0.4) (layer "F.Cu") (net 15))
 (segment (start 108.1788 107.6836) (end 108.1788 107.1248) (width 0.4) (layer "F.Cu") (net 15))
 (segment (start 116.1544 125.7684) (end 116.1544 131.3056) (width 0.4) (layer "F.Cu") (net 15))
 (segment (start 116.6116 131.7628) (end 116.6116 138.57) (width 0.4) (layer "F.Cu") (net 15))
 (segment (start 108.1788 116.1672) (end 116.1544 124.1428) (width 0.4) (layer "F.Cu") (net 15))
 (via (at 108.1788 107.6836) (size 1.5) (drill 0.5) (layers "F.Cu" "B.Cu") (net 15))
 (via (at 108.1788 110.9348) (size 1.5) (drill 0.5) (layers "F.Cu" "B.Cu") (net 15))
 (segment (start 108.1788 107.6836) (end 108.1788 110.9348) (width 0.4) (layer "B.Cu") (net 15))
 (segment (start 107.6384 109.1892) (end 110.4104 109.1892) (width 0.4) (layer "F.Cu") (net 10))
 (segment (start 117.4244 140.602) (end 118.8468 140.602) (width 0.4) (layer "F.Cu") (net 10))
 (segment (start 115.8496 139.0272) (end 117.4244 140.602) (width 0.4) (layer "F.Cu") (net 10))
 (segment (start 106.604 116.8784) (end 106.604 110.2236) (width 0.4) (layer "F.Cu") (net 10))
 (segment (start 113.6144 131.3056) (end 115.8496 133.5408) (width 0.4) (layer "F.Cu") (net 10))
 (segment (start 119.431 141.1862) (end 119.431 142.315) (width 0.4) (layer "F.Cu") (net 10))
 (segment (start 113.6144 123.8888) (end 106.604 116.8784) (width 0.4) (layer "F.Cu") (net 10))
 (segment (start 115.8496 133.5408) (end 115.8496 139.0272) (width 0.4) (layer "F.Cu") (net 10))
 (segment (start 113.6144 125.7684) (end 113.6144 131.3056) (width 0.4) (layer "F.Cu") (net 10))
 (segment (start 106.604 110.2236) (end 107.6384 109.1892) (width 0.4) (layer "F.Cu") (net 10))
 (segment (start 113.6144 125.7684) (end 113.6144 123.8888) (width 0.4) (layer "F.Cu") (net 10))
 (segment (start 118.8468 140.602) (end 119.431 141.1862) (width 0.4) (layer "F.Cu") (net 10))
 (segment (start 115.5208 106.192) (end 115.5448 106.168) (width 0.4) (layer "F.Cu") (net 21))
 (segment (start 112.4104 106.192) (end 115.5208 106.192) (width 0.4) (layer "F.Cu") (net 21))
 (segment (start 112.4104 109.1892) (end 115.5236 109.1892) (width 0.4) (layer "F.Cu") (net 11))
 (segment (start 115.5236 109.1892) (end 115.5448 109.168) (width 0.4) (layer "F.Cu") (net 11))
 (segment (start 113.956 112.168) (end 113.0556 113.0684) (width 0.4) (layer "F.Cu") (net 2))
 (segment (start 115.3416 117.2848) (end 118.5232 117.2848) (width 0.4) (layer "F.Cu") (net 2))
 (segment (start 113.0556 113.0684) (end 113.0556 114.9988) (width 0.4) (layer "F.Cu") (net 2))
 (segment (start 115.5448 112.168) (end 113.956 112.168) (width 0.4) (layer "F.Cu") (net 2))
 (segment (start 118.5232 117.2848) (end 118.542 117.266) (width 0.4) (layer "F.Cu") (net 2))
 (segment (start 113.0556 114.9988) (end 115.3416 117.2848) (width 0.4) (layer "F.Cu") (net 2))
 (segment (start 135.0448 109.168) (end 138.2088 109.168) (width 0.4) (layer "F.Cu") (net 5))
 (segment (start 138.2088 109.168) (end 138.23 109.1892) (width 0.4) (layer "F.Cu") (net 5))
 (segment (start 135.0448 112.168) (end 138.2116 112.168) (width 0.4) (layer "F.Cu") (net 7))
 (segment (start 138.2116 112.168) (end 138.23 112.1864) (width 0.4) (layer "F.Cu") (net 7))
 (segment (start 133.3728 100.168) (end 132.258 101.2828) (width 0.4) (layer "F.Cu") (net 16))
 (segment (start 131.0068 117.1644) (end 121.1328 117.1644) (width 0.4) (layer "F.Cu") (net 16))
 (segment (start 132.258 115.9132) (end 131.0068 117.1644) (width 0.4) (layer "F.Cu") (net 16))
 (segment (start 132.258 101.2828) (end 132.258 115.9132) (width 0.4) (layer "F.Cu") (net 16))
 (segment (start 135.0448 100.168) (end 133.3728 100.168) (width 0.4) (layer "F.Cu") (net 16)))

